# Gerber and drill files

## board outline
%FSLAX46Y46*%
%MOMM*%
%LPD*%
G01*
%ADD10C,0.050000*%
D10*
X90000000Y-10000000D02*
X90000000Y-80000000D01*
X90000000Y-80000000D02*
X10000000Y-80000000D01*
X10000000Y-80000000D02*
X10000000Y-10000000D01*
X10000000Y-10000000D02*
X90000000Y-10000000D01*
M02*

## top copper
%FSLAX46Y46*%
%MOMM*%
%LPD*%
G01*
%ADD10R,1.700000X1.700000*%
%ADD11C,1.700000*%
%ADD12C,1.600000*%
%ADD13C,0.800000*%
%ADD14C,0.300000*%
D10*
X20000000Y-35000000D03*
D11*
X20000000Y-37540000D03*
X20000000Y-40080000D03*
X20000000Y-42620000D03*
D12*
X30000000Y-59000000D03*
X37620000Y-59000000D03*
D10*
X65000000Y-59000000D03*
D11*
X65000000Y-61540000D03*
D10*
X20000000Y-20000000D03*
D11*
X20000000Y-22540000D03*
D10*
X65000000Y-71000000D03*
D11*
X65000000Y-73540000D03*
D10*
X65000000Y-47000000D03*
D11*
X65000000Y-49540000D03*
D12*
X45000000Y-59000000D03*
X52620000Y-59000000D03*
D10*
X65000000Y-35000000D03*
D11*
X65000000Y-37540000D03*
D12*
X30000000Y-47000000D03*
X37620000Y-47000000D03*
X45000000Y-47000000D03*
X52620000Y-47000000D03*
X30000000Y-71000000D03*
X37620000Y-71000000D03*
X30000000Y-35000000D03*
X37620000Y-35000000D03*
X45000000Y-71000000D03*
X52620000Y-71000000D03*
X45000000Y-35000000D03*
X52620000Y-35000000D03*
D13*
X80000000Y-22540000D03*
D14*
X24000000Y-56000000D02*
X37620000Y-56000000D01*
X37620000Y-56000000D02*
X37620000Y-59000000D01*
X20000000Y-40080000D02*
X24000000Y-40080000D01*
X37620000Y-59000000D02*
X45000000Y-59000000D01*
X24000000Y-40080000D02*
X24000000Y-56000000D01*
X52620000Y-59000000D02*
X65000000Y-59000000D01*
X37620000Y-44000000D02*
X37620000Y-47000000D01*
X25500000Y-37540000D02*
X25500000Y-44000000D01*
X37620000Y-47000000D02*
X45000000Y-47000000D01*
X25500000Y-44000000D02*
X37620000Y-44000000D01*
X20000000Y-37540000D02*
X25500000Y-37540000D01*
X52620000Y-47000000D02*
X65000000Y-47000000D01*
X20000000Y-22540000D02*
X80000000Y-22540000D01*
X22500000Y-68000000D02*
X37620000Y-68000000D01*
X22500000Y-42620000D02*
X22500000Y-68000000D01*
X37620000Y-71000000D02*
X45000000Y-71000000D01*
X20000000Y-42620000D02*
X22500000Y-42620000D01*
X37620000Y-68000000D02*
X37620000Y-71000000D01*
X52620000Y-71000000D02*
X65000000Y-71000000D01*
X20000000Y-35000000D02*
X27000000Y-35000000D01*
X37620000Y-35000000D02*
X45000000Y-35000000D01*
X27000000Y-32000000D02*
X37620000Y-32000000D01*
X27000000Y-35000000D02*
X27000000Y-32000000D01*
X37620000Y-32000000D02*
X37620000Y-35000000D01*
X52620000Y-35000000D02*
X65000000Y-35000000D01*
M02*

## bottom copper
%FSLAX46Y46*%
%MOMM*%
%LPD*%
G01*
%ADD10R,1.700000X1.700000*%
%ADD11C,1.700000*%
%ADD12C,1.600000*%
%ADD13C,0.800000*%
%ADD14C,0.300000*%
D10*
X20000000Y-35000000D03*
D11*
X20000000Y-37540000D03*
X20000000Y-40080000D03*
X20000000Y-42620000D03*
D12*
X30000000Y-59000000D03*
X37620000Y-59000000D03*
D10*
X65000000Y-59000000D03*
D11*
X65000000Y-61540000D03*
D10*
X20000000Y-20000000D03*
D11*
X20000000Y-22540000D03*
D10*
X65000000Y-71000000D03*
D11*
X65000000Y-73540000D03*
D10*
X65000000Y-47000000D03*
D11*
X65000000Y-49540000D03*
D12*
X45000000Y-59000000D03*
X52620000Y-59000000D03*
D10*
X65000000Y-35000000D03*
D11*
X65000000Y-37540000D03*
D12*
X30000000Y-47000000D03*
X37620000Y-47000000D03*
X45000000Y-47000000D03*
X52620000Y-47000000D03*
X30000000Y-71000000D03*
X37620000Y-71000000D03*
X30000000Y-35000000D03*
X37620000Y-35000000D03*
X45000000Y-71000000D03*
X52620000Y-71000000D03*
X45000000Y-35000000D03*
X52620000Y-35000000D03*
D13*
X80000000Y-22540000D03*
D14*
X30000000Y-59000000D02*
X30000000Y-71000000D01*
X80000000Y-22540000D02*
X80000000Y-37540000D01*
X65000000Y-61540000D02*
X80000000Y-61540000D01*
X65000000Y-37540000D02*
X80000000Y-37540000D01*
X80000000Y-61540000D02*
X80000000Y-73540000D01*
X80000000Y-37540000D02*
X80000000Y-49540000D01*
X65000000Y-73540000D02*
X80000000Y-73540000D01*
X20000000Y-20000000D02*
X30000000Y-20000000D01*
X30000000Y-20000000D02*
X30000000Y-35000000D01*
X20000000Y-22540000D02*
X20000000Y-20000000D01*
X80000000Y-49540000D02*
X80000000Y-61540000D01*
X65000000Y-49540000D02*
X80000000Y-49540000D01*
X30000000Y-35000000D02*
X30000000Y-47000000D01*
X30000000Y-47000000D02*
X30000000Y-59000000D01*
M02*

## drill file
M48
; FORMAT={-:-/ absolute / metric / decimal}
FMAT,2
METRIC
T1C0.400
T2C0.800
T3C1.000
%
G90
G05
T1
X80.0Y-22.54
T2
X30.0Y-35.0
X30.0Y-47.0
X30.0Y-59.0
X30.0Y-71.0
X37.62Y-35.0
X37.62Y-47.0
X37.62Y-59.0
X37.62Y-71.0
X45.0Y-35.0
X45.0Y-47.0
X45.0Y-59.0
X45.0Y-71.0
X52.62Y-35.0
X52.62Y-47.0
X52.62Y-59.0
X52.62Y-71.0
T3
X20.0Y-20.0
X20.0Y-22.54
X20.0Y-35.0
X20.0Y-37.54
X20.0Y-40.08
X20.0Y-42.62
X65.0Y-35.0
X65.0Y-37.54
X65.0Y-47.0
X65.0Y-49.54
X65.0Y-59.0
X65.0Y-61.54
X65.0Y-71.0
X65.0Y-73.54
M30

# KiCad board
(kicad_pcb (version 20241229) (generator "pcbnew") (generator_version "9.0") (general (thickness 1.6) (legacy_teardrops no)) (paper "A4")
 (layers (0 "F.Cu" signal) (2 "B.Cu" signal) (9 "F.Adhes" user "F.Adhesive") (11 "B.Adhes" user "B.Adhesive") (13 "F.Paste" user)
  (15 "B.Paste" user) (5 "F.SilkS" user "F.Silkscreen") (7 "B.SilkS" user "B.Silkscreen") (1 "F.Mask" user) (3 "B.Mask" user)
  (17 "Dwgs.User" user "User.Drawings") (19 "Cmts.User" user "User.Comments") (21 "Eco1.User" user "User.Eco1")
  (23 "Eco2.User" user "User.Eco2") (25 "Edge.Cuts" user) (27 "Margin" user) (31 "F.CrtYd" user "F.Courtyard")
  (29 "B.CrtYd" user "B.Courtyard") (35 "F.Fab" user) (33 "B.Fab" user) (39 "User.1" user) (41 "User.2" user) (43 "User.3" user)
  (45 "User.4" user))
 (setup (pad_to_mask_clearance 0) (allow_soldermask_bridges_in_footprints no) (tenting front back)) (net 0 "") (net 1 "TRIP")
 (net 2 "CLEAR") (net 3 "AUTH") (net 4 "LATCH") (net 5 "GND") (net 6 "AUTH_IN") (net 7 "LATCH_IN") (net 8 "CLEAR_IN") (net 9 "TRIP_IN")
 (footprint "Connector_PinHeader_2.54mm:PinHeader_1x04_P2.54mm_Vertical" (layer "F.Cu") (at 20 35)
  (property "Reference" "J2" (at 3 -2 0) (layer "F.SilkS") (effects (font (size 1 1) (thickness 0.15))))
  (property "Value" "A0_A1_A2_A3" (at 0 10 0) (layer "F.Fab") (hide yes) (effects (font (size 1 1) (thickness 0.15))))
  (pad "1" thru_hole rect (at 0 0) (size 1.7 1.7) (drill 1) (layers "*.Cu" "*.Mask") (remove_unused_layers no) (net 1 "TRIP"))
  (pad "2" thru_hole circle (at 0 2.54) (size 1.7 1.7) (drill 1) (layers "*.Cu" "*.Mask") (remove_unused_layers no) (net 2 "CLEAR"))
  (pad "3" thru_hole circle (at 0 5.08) (size 1.7 1.7) (drill 1) (layers "*.Cu" "*.Mask") (remove_unused_layers no) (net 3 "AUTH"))
  (pad "4" thru_hole circle (at 0 7.62) (size 1.7 1.7) (drill 1) (layers "*.Cu" "*.Mask") (remove_unused_layers no) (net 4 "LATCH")))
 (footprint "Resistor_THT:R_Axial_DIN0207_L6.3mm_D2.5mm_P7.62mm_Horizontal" (layer "F.Cu") (at 30 59)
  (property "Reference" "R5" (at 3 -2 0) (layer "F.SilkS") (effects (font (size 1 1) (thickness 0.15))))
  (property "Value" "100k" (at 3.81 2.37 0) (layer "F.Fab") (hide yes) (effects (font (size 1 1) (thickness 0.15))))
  (pad "1" thru_hole circle (at 0 0) (size 1.6 1.6) (drill 0.8) (layers "*.Cu" "*.Mask") (remove_unused_layers no) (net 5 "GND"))
  (pad "2" thru_hole circle (at 7.62 0) (size 1.6 1.6) (drill 0.8) (layers "*.Cu" "*.Mask") (remove_unused_layers no) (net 3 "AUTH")))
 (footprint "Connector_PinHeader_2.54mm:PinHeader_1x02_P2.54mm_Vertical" (layer "F.Cu") (at 65 59)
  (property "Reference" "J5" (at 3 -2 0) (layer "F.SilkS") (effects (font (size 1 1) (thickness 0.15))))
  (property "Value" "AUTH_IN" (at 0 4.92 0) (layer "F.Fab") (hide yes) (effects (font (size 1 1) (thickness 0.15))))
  (pad "1" thru_hole rect (at 0 0) (size 1.7 1.7) (drill 1) (layers "*.Cu" "*.Mask") (remove_unused_layers no) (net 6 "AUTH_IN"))
  (pad "2" thru_hole circle (at 0 2.54) (size 1.7 1.7) (drill 1) (layers "*.Cu" "*.Mask") (remove_unused_layers no) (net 5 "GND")))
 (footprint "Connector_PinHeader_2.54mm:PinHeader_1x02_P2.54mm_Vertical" (layer "F.Cu") (at 20 20)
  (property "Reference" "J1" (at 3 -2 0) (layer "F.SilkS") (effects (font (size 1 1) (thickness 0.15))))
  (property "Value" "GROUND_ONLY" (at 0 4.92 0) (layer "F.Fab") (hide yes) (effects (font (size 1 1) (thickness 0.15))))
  (pad "1" thru_hole rect (at 0 0) (size 1.7 1.7) (drill 1) (layers "*.Cu" "*.Mask") (remove_unused_layers no) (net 5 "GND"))
  (pad "2" thru_hole circle (at 0 2.54) (size 1.7 1.7) (drill 1) (layers "*.Cu" "*.Mask") (remove_unused_layers no) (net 5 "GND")))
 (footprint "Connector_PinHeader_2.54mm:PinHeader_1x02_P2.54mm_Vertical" (layer "F.Cu") (at 65 71)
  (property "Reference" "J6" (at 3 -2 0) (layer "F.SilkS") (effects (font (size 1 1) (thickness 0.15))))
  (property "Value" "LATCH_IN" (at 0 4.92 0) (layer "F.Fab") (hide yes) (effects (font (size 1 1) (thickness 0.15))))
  (pad "1" thru_hole rect (at 0 0) (size 1.7 1.7) (drill 1) (layers "*.Cu" "*.Mask") (remove_unused_layers no) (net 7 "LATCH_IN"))
  (pad "2" thru_hole circle (at 0 2.54) (size 1.7 1.7) (drill 1) (layers "*.Cu" "*.Mask") (remove_unused_layers no) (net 5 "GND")))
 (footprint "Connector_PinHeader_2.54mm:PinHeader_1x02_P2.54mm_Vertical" (layer "F.Cu") (at 65 47)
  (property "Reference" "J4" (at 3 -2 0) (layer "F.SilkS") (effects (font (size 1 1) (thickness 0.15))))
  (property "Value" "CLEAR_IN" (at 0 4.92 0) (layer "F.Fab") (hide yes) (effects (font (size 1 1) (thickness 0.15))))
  (pad "1" thru_hole rect (at 0 0) (size 1.7 1.7) (drill 1) (layers "*.Cu" "*.Mask") (remove_unused_layers no) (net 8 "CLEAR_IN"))
  (pad "2" thru_hole circle (at 0 2.54) (size 1.7 1.7) (drill 1) (layers "*.Cu" "*.Mask") (remove_unused_layers no) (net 5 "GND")))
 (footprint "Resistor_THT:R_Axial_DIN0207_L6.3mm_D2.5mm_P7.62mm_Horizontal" (layer "F.Cu") (at 45 59)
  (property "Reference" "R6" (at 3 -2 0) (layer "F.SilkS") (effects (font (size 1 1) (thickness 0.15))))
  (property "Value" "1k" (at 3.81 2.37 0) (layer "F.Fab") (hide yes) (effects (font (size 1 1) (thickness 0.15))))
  (pad "1" thru_hole circle (at 0 0) (size 1.6 1.6) (drill 0.8) (layers "*.Cu" "*.Mask") (remove_unused_layers no) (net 3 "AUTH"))
  (pad "2" thru_hole circle (at 7.62 0) (size 1.6 1.6) (drill 0.8) (layers "*.Cu" "*.Mask") (remove_unused_layers no) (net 6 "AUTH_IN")))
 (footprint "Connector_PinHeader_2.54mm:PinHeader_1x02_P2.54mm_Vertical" (layer "F.Cu") (at 65 35)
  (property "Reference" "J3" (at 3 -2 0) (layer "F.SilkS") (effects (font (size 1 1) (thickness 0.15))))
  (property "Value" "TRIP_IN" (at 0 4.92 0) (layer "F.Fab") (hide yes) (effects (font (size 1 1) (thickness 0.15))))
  (pad "1" thru_hole rect (at 0 0) (size 1.7 1.7) (drill 1) (layers "*.Cu" "*.Mask") (remove_unused_layers no) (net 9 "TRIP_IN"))
  (pad "2" thru_hole circle (at 0 2.54) (size 1.7 1.7) (drill 1) (layers "*.Cu" "*.Mask") (remove_unused_layers no) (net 5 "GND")))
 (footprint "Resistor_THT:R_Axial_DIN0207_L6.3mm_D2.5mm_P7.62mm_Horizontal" (layer "F.Cu") (at 30 47)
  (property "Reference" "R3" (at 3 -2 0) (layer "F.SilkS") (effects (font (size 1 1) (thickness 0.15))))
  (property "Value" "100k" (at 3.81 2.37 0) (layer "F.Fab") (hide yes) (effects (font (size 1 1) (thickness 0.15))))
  (pad "1" thru_hole circle (at 0 0) (size 1.6 1.6) (drill 0.8) (layers "*.Cu" "*.Mask") (remove_unused_layers no) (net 5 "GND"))
  (pad "2" thru_hole circle (at 7.62 0) (size 1.6 1.6) (drill 0.8) (layers "*.Cu" "*.Mask") (remove_unused_layers no) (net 2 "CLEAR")))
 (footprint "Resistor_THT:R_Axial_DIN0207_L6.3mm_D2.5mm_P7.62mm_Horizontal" (layer "F.Cu") (at 45 47)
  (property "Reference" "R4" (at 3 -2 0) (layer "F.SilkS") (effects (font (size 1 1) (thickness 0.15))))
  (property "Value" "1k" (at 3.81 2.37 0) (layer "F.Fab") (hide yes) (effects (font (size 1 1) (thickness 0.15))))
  (pad "1" thru_hole circle (at 0 0) (size 1.6 1.6) (drill 0.8) (layers "*.Cu" "*.Mask") (remove_unused_layers no) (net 2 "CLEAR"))
  (pad "2" thru_hole circle (at 7.62 0) (size 1.6 1.6) (drill 0.8) (layers "*.Cu" "*.Mask") (remove_unused_layers no) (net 8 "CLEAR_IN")))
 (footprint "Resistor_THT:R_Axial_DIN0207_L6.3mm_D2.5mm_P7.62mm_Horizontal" (layer "F.Cu") (at 30 71)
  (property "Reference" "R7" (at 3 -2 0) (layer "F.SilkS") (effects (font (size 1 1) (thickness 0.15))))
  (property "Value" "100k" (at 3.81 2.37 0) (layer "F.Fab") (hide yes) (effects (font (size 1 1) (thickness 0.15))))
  (pad "1" thru_hole circle (at 0 0) (size 1.6 1.6) (drill 0.8) (layers "*.Cu" "*.Mask") (remove_unused_layers no) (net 5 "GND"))
  (pad "2" thru_hole circle (at 7.62 0) (size 1.6 1.6) (drill 0.8) (layers "*.Cu" "*.Mask") (remove_unused_layers no) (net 4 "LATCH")))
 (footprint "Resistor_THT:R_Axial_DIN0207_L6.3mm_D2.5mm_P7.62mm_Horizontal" (layer "F.Cu") (at 30 35)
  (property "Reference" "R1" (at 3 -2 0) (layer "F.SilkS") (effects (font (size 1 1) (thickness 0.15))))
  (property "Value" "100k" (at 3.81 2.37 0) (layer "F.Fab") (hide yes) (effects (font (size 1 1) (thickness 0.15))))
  (pad "1" thru_hole circle (at 0 0) (size 1.6 1.6) (drill 0.8) (layers "*.Cu" "*.Mask") (remove_unused_layers no) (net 5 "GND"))
  (pad "2" thru_hole circle (at 7.62 0) (size 1.6 1.6) (drill 0.8) (layers "*.Cu" "*.Mask") (remove_unused_layers no) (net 1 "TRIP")))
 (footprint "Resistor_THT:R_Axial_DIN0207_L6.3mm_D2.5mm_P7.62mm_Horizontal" (layer "F.Cu") (at 45 71)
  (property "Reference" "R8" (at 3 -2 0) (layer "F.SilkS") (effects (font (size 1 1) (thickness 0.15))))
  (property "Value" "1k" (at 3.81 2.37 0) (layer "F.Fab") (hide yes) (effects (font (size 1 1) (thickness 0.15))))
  (pad "1" thru_hole circle (at 0 0) (size 1.6 1.6) (drill 0.8) (layers "*.Cu" "*.Mask") (remove_unused_layers no) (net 4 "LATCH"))
  (pad "2" thru_hole circle (at 7.62 0) (size 1.6 1.6) (drill 0.8) (layers "*.Cu" "*.Mask") (remove_unused_layers no) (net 7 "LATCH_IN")))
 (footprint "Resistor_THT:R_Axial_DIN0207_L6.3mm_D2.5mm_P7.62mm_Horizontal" (layer "F.Cu") (at 45 35)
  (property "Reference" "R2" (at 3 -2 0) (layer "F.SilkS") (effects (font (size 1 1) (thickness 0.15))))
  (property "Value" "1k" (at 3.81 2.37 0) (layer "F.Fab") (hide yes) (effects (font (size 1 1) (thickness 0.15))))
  (pad "1" thru_hole circle (at 0 0) (size 1.6 1.6) (drill 0.8) (layers "*.Cu" "*.Mask") (remove_unused_layers no) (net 1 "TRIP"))
  (pad "2" thru_hole circle (at 7.62 0) (size 1.6 1.6) (drill 0.8) (layers "*.Cu" "*.Mask") (remove_unused_layers no) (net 9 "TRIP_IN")))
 (gr_line (start 90 10) (end 90 80) (stroke (width 0.05) (type default)) (layer "Edge.Cuts"))
 (gr_line (start 90 80) (end 10 80) (stroke (width 0.05) (type default)) (layer "Edge.Cuts"))
 (gr_line (start 10 80) (end 10 10) (stroke (width 0.05) (type default)) (layer "Edge.Cuts"))
 (gr_line (start 10 10) (end 90 10) (stroke (width 0.05) (type default)) (layer "Edge.Cuts"))
 (segment (start 24 56) (end 37.62 56) (width 0.3) (layer "F.Cu") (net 3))
 (segment (start 37.62 56) (end 37.62 59) (width 0.3) (layer "F.Cu") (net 3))
 (segment (start 20 40.08) (end 24 40.08) (width 0.3) (layer "F.Cu") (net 3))
 (segment (start 37.62 59) (end 45 59) (width 0.3) (layer "F.Cu") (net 3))
 (segment (start 24 40.08) (end 24 56) (width 0.3) (layer "F.Cu") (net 3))
 (segment (start 52.62 59) (end 65 59) (width 0.3) (layer "F.Cu") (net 6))
 (segment (start 37.62 44) (end 37.62 47) (width 0.3) (layer "F.Cu") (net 2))
 (segment (start 25.5 37.54) (end 25.5 44) (width 0.3) (layer "F.Cu") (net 2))
 (segment (start 37.62 47) (end 45 47) (width 0.3) (layer "F.Cu") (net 2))
 (segment (start 25.5 44) (end 37.62 44) (width 0.3) (layer "F.Cu") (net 2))
 (segment (start 20 37.54) (end 25.5 37.54) (width 0.3) (layer "F.Cu") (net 2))
 (segment (start 52.62 47) (end 65 47) (width 0.3) (layer "F.Cu") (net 8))
 (segment (start 20 22.54) (end 80 22.54) (width 0.3) (layer "F.Cu") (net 5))
 (via (at 80 22.54) (size 0.8) (drill 0.4) (layers "F.Cu" "B.Cu") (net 5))
 (segment (start 30 59) (end 30 71) (width 0.3) (layer "B.Cu") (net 5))
 (segment (start 80 22.54) (end 80 37.54) (width 0.3) (layer "B.Cu") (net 5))
 (segment (start 65 61.54) (end 80 61.54) (width 0.3) (layer "B.Cu") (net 5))
 (segment (start 65 37.54) (end 80 37.54) (width 0.3) (layer "B.Cu") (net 5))
 (segment (start 80 61.54) (end 80 73.54) (width 0.3) (layer "B.Cu") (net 5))
 (segment (start 80 37.54) (end 80 49.54) (width 0.3) (layer "B.Cu") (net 5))
 (segment (start 65 73.54) (end 80 73.54) (width 0.3) (layer "B.Cu") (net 5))
 (segment (start 20 20) (end 30 20) (width 0.3) (layer "B.Cu") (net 5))
 (segment (start 30 20) (end 30 35) (width 0.3) (layer "B.Cu") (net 5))
 (segment (start 20 22.54) (end 20 20) (width 0.3) (layer "B.Cu") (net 5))
 (segment (start 80 49.54) (end 80 61.54) (width 0.3) (layer "B.Cu") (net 5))
 (segment (start 65 49.54) (end 80 49.54) (width 0.3) (layer "B.Cu") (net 5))
 (segment (start 30 35) (end 30 47) (width 0.3) (layer "B.Cu") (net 5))
 (segment (start 30 47) (end 30 59) (width 0.3) (layer "B.Cu") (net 5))
 (segment (start 22.5 68) (end 37.62 68) (width 0.3) (layer "F.Cu") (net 4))
 (segment (start 22.5 42.62) (end 22.5 68) (width 0.3) (layer "F.Cu") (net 4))
 (segment (start 37.62 71) (end 45 71) (width 0.3) (layer "F.Cu") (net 4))
 (segment (start 20 42.62) (end 22.5 42.62) (width 0.3) (layer "F.Cu") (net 4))
 (segment (start 37.62 68) (end 37.62 71) (width 0.3) (layer "F.Cu") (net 4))
 (segment (start 52.62 71) (end 65 71) (width 0.3) (layer "F.Cu") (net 7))
 (segment (start 20 35) (end 27 35) (width 0.3) (layer "F.Cu") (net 1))
 (segment (start 37.62 35) (end 45 35) (width 0.3) (layer "F.Cu") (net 1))
 (segment (start 27 32) (end 37.62 32) (width 0.3) (layer "F.Cu") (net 1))
 (segment (start 27 35) (end 27 32) (width 0.3) (layer "F.Cu") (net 1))
 (segment (start 37.62 32) (end 37.62 35) (width 0.3) (layer "F.Cu") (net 1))
 (segment (start 52.62 35) (end 65 35) (width 0.3) (layer "F.Cu") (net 9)))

